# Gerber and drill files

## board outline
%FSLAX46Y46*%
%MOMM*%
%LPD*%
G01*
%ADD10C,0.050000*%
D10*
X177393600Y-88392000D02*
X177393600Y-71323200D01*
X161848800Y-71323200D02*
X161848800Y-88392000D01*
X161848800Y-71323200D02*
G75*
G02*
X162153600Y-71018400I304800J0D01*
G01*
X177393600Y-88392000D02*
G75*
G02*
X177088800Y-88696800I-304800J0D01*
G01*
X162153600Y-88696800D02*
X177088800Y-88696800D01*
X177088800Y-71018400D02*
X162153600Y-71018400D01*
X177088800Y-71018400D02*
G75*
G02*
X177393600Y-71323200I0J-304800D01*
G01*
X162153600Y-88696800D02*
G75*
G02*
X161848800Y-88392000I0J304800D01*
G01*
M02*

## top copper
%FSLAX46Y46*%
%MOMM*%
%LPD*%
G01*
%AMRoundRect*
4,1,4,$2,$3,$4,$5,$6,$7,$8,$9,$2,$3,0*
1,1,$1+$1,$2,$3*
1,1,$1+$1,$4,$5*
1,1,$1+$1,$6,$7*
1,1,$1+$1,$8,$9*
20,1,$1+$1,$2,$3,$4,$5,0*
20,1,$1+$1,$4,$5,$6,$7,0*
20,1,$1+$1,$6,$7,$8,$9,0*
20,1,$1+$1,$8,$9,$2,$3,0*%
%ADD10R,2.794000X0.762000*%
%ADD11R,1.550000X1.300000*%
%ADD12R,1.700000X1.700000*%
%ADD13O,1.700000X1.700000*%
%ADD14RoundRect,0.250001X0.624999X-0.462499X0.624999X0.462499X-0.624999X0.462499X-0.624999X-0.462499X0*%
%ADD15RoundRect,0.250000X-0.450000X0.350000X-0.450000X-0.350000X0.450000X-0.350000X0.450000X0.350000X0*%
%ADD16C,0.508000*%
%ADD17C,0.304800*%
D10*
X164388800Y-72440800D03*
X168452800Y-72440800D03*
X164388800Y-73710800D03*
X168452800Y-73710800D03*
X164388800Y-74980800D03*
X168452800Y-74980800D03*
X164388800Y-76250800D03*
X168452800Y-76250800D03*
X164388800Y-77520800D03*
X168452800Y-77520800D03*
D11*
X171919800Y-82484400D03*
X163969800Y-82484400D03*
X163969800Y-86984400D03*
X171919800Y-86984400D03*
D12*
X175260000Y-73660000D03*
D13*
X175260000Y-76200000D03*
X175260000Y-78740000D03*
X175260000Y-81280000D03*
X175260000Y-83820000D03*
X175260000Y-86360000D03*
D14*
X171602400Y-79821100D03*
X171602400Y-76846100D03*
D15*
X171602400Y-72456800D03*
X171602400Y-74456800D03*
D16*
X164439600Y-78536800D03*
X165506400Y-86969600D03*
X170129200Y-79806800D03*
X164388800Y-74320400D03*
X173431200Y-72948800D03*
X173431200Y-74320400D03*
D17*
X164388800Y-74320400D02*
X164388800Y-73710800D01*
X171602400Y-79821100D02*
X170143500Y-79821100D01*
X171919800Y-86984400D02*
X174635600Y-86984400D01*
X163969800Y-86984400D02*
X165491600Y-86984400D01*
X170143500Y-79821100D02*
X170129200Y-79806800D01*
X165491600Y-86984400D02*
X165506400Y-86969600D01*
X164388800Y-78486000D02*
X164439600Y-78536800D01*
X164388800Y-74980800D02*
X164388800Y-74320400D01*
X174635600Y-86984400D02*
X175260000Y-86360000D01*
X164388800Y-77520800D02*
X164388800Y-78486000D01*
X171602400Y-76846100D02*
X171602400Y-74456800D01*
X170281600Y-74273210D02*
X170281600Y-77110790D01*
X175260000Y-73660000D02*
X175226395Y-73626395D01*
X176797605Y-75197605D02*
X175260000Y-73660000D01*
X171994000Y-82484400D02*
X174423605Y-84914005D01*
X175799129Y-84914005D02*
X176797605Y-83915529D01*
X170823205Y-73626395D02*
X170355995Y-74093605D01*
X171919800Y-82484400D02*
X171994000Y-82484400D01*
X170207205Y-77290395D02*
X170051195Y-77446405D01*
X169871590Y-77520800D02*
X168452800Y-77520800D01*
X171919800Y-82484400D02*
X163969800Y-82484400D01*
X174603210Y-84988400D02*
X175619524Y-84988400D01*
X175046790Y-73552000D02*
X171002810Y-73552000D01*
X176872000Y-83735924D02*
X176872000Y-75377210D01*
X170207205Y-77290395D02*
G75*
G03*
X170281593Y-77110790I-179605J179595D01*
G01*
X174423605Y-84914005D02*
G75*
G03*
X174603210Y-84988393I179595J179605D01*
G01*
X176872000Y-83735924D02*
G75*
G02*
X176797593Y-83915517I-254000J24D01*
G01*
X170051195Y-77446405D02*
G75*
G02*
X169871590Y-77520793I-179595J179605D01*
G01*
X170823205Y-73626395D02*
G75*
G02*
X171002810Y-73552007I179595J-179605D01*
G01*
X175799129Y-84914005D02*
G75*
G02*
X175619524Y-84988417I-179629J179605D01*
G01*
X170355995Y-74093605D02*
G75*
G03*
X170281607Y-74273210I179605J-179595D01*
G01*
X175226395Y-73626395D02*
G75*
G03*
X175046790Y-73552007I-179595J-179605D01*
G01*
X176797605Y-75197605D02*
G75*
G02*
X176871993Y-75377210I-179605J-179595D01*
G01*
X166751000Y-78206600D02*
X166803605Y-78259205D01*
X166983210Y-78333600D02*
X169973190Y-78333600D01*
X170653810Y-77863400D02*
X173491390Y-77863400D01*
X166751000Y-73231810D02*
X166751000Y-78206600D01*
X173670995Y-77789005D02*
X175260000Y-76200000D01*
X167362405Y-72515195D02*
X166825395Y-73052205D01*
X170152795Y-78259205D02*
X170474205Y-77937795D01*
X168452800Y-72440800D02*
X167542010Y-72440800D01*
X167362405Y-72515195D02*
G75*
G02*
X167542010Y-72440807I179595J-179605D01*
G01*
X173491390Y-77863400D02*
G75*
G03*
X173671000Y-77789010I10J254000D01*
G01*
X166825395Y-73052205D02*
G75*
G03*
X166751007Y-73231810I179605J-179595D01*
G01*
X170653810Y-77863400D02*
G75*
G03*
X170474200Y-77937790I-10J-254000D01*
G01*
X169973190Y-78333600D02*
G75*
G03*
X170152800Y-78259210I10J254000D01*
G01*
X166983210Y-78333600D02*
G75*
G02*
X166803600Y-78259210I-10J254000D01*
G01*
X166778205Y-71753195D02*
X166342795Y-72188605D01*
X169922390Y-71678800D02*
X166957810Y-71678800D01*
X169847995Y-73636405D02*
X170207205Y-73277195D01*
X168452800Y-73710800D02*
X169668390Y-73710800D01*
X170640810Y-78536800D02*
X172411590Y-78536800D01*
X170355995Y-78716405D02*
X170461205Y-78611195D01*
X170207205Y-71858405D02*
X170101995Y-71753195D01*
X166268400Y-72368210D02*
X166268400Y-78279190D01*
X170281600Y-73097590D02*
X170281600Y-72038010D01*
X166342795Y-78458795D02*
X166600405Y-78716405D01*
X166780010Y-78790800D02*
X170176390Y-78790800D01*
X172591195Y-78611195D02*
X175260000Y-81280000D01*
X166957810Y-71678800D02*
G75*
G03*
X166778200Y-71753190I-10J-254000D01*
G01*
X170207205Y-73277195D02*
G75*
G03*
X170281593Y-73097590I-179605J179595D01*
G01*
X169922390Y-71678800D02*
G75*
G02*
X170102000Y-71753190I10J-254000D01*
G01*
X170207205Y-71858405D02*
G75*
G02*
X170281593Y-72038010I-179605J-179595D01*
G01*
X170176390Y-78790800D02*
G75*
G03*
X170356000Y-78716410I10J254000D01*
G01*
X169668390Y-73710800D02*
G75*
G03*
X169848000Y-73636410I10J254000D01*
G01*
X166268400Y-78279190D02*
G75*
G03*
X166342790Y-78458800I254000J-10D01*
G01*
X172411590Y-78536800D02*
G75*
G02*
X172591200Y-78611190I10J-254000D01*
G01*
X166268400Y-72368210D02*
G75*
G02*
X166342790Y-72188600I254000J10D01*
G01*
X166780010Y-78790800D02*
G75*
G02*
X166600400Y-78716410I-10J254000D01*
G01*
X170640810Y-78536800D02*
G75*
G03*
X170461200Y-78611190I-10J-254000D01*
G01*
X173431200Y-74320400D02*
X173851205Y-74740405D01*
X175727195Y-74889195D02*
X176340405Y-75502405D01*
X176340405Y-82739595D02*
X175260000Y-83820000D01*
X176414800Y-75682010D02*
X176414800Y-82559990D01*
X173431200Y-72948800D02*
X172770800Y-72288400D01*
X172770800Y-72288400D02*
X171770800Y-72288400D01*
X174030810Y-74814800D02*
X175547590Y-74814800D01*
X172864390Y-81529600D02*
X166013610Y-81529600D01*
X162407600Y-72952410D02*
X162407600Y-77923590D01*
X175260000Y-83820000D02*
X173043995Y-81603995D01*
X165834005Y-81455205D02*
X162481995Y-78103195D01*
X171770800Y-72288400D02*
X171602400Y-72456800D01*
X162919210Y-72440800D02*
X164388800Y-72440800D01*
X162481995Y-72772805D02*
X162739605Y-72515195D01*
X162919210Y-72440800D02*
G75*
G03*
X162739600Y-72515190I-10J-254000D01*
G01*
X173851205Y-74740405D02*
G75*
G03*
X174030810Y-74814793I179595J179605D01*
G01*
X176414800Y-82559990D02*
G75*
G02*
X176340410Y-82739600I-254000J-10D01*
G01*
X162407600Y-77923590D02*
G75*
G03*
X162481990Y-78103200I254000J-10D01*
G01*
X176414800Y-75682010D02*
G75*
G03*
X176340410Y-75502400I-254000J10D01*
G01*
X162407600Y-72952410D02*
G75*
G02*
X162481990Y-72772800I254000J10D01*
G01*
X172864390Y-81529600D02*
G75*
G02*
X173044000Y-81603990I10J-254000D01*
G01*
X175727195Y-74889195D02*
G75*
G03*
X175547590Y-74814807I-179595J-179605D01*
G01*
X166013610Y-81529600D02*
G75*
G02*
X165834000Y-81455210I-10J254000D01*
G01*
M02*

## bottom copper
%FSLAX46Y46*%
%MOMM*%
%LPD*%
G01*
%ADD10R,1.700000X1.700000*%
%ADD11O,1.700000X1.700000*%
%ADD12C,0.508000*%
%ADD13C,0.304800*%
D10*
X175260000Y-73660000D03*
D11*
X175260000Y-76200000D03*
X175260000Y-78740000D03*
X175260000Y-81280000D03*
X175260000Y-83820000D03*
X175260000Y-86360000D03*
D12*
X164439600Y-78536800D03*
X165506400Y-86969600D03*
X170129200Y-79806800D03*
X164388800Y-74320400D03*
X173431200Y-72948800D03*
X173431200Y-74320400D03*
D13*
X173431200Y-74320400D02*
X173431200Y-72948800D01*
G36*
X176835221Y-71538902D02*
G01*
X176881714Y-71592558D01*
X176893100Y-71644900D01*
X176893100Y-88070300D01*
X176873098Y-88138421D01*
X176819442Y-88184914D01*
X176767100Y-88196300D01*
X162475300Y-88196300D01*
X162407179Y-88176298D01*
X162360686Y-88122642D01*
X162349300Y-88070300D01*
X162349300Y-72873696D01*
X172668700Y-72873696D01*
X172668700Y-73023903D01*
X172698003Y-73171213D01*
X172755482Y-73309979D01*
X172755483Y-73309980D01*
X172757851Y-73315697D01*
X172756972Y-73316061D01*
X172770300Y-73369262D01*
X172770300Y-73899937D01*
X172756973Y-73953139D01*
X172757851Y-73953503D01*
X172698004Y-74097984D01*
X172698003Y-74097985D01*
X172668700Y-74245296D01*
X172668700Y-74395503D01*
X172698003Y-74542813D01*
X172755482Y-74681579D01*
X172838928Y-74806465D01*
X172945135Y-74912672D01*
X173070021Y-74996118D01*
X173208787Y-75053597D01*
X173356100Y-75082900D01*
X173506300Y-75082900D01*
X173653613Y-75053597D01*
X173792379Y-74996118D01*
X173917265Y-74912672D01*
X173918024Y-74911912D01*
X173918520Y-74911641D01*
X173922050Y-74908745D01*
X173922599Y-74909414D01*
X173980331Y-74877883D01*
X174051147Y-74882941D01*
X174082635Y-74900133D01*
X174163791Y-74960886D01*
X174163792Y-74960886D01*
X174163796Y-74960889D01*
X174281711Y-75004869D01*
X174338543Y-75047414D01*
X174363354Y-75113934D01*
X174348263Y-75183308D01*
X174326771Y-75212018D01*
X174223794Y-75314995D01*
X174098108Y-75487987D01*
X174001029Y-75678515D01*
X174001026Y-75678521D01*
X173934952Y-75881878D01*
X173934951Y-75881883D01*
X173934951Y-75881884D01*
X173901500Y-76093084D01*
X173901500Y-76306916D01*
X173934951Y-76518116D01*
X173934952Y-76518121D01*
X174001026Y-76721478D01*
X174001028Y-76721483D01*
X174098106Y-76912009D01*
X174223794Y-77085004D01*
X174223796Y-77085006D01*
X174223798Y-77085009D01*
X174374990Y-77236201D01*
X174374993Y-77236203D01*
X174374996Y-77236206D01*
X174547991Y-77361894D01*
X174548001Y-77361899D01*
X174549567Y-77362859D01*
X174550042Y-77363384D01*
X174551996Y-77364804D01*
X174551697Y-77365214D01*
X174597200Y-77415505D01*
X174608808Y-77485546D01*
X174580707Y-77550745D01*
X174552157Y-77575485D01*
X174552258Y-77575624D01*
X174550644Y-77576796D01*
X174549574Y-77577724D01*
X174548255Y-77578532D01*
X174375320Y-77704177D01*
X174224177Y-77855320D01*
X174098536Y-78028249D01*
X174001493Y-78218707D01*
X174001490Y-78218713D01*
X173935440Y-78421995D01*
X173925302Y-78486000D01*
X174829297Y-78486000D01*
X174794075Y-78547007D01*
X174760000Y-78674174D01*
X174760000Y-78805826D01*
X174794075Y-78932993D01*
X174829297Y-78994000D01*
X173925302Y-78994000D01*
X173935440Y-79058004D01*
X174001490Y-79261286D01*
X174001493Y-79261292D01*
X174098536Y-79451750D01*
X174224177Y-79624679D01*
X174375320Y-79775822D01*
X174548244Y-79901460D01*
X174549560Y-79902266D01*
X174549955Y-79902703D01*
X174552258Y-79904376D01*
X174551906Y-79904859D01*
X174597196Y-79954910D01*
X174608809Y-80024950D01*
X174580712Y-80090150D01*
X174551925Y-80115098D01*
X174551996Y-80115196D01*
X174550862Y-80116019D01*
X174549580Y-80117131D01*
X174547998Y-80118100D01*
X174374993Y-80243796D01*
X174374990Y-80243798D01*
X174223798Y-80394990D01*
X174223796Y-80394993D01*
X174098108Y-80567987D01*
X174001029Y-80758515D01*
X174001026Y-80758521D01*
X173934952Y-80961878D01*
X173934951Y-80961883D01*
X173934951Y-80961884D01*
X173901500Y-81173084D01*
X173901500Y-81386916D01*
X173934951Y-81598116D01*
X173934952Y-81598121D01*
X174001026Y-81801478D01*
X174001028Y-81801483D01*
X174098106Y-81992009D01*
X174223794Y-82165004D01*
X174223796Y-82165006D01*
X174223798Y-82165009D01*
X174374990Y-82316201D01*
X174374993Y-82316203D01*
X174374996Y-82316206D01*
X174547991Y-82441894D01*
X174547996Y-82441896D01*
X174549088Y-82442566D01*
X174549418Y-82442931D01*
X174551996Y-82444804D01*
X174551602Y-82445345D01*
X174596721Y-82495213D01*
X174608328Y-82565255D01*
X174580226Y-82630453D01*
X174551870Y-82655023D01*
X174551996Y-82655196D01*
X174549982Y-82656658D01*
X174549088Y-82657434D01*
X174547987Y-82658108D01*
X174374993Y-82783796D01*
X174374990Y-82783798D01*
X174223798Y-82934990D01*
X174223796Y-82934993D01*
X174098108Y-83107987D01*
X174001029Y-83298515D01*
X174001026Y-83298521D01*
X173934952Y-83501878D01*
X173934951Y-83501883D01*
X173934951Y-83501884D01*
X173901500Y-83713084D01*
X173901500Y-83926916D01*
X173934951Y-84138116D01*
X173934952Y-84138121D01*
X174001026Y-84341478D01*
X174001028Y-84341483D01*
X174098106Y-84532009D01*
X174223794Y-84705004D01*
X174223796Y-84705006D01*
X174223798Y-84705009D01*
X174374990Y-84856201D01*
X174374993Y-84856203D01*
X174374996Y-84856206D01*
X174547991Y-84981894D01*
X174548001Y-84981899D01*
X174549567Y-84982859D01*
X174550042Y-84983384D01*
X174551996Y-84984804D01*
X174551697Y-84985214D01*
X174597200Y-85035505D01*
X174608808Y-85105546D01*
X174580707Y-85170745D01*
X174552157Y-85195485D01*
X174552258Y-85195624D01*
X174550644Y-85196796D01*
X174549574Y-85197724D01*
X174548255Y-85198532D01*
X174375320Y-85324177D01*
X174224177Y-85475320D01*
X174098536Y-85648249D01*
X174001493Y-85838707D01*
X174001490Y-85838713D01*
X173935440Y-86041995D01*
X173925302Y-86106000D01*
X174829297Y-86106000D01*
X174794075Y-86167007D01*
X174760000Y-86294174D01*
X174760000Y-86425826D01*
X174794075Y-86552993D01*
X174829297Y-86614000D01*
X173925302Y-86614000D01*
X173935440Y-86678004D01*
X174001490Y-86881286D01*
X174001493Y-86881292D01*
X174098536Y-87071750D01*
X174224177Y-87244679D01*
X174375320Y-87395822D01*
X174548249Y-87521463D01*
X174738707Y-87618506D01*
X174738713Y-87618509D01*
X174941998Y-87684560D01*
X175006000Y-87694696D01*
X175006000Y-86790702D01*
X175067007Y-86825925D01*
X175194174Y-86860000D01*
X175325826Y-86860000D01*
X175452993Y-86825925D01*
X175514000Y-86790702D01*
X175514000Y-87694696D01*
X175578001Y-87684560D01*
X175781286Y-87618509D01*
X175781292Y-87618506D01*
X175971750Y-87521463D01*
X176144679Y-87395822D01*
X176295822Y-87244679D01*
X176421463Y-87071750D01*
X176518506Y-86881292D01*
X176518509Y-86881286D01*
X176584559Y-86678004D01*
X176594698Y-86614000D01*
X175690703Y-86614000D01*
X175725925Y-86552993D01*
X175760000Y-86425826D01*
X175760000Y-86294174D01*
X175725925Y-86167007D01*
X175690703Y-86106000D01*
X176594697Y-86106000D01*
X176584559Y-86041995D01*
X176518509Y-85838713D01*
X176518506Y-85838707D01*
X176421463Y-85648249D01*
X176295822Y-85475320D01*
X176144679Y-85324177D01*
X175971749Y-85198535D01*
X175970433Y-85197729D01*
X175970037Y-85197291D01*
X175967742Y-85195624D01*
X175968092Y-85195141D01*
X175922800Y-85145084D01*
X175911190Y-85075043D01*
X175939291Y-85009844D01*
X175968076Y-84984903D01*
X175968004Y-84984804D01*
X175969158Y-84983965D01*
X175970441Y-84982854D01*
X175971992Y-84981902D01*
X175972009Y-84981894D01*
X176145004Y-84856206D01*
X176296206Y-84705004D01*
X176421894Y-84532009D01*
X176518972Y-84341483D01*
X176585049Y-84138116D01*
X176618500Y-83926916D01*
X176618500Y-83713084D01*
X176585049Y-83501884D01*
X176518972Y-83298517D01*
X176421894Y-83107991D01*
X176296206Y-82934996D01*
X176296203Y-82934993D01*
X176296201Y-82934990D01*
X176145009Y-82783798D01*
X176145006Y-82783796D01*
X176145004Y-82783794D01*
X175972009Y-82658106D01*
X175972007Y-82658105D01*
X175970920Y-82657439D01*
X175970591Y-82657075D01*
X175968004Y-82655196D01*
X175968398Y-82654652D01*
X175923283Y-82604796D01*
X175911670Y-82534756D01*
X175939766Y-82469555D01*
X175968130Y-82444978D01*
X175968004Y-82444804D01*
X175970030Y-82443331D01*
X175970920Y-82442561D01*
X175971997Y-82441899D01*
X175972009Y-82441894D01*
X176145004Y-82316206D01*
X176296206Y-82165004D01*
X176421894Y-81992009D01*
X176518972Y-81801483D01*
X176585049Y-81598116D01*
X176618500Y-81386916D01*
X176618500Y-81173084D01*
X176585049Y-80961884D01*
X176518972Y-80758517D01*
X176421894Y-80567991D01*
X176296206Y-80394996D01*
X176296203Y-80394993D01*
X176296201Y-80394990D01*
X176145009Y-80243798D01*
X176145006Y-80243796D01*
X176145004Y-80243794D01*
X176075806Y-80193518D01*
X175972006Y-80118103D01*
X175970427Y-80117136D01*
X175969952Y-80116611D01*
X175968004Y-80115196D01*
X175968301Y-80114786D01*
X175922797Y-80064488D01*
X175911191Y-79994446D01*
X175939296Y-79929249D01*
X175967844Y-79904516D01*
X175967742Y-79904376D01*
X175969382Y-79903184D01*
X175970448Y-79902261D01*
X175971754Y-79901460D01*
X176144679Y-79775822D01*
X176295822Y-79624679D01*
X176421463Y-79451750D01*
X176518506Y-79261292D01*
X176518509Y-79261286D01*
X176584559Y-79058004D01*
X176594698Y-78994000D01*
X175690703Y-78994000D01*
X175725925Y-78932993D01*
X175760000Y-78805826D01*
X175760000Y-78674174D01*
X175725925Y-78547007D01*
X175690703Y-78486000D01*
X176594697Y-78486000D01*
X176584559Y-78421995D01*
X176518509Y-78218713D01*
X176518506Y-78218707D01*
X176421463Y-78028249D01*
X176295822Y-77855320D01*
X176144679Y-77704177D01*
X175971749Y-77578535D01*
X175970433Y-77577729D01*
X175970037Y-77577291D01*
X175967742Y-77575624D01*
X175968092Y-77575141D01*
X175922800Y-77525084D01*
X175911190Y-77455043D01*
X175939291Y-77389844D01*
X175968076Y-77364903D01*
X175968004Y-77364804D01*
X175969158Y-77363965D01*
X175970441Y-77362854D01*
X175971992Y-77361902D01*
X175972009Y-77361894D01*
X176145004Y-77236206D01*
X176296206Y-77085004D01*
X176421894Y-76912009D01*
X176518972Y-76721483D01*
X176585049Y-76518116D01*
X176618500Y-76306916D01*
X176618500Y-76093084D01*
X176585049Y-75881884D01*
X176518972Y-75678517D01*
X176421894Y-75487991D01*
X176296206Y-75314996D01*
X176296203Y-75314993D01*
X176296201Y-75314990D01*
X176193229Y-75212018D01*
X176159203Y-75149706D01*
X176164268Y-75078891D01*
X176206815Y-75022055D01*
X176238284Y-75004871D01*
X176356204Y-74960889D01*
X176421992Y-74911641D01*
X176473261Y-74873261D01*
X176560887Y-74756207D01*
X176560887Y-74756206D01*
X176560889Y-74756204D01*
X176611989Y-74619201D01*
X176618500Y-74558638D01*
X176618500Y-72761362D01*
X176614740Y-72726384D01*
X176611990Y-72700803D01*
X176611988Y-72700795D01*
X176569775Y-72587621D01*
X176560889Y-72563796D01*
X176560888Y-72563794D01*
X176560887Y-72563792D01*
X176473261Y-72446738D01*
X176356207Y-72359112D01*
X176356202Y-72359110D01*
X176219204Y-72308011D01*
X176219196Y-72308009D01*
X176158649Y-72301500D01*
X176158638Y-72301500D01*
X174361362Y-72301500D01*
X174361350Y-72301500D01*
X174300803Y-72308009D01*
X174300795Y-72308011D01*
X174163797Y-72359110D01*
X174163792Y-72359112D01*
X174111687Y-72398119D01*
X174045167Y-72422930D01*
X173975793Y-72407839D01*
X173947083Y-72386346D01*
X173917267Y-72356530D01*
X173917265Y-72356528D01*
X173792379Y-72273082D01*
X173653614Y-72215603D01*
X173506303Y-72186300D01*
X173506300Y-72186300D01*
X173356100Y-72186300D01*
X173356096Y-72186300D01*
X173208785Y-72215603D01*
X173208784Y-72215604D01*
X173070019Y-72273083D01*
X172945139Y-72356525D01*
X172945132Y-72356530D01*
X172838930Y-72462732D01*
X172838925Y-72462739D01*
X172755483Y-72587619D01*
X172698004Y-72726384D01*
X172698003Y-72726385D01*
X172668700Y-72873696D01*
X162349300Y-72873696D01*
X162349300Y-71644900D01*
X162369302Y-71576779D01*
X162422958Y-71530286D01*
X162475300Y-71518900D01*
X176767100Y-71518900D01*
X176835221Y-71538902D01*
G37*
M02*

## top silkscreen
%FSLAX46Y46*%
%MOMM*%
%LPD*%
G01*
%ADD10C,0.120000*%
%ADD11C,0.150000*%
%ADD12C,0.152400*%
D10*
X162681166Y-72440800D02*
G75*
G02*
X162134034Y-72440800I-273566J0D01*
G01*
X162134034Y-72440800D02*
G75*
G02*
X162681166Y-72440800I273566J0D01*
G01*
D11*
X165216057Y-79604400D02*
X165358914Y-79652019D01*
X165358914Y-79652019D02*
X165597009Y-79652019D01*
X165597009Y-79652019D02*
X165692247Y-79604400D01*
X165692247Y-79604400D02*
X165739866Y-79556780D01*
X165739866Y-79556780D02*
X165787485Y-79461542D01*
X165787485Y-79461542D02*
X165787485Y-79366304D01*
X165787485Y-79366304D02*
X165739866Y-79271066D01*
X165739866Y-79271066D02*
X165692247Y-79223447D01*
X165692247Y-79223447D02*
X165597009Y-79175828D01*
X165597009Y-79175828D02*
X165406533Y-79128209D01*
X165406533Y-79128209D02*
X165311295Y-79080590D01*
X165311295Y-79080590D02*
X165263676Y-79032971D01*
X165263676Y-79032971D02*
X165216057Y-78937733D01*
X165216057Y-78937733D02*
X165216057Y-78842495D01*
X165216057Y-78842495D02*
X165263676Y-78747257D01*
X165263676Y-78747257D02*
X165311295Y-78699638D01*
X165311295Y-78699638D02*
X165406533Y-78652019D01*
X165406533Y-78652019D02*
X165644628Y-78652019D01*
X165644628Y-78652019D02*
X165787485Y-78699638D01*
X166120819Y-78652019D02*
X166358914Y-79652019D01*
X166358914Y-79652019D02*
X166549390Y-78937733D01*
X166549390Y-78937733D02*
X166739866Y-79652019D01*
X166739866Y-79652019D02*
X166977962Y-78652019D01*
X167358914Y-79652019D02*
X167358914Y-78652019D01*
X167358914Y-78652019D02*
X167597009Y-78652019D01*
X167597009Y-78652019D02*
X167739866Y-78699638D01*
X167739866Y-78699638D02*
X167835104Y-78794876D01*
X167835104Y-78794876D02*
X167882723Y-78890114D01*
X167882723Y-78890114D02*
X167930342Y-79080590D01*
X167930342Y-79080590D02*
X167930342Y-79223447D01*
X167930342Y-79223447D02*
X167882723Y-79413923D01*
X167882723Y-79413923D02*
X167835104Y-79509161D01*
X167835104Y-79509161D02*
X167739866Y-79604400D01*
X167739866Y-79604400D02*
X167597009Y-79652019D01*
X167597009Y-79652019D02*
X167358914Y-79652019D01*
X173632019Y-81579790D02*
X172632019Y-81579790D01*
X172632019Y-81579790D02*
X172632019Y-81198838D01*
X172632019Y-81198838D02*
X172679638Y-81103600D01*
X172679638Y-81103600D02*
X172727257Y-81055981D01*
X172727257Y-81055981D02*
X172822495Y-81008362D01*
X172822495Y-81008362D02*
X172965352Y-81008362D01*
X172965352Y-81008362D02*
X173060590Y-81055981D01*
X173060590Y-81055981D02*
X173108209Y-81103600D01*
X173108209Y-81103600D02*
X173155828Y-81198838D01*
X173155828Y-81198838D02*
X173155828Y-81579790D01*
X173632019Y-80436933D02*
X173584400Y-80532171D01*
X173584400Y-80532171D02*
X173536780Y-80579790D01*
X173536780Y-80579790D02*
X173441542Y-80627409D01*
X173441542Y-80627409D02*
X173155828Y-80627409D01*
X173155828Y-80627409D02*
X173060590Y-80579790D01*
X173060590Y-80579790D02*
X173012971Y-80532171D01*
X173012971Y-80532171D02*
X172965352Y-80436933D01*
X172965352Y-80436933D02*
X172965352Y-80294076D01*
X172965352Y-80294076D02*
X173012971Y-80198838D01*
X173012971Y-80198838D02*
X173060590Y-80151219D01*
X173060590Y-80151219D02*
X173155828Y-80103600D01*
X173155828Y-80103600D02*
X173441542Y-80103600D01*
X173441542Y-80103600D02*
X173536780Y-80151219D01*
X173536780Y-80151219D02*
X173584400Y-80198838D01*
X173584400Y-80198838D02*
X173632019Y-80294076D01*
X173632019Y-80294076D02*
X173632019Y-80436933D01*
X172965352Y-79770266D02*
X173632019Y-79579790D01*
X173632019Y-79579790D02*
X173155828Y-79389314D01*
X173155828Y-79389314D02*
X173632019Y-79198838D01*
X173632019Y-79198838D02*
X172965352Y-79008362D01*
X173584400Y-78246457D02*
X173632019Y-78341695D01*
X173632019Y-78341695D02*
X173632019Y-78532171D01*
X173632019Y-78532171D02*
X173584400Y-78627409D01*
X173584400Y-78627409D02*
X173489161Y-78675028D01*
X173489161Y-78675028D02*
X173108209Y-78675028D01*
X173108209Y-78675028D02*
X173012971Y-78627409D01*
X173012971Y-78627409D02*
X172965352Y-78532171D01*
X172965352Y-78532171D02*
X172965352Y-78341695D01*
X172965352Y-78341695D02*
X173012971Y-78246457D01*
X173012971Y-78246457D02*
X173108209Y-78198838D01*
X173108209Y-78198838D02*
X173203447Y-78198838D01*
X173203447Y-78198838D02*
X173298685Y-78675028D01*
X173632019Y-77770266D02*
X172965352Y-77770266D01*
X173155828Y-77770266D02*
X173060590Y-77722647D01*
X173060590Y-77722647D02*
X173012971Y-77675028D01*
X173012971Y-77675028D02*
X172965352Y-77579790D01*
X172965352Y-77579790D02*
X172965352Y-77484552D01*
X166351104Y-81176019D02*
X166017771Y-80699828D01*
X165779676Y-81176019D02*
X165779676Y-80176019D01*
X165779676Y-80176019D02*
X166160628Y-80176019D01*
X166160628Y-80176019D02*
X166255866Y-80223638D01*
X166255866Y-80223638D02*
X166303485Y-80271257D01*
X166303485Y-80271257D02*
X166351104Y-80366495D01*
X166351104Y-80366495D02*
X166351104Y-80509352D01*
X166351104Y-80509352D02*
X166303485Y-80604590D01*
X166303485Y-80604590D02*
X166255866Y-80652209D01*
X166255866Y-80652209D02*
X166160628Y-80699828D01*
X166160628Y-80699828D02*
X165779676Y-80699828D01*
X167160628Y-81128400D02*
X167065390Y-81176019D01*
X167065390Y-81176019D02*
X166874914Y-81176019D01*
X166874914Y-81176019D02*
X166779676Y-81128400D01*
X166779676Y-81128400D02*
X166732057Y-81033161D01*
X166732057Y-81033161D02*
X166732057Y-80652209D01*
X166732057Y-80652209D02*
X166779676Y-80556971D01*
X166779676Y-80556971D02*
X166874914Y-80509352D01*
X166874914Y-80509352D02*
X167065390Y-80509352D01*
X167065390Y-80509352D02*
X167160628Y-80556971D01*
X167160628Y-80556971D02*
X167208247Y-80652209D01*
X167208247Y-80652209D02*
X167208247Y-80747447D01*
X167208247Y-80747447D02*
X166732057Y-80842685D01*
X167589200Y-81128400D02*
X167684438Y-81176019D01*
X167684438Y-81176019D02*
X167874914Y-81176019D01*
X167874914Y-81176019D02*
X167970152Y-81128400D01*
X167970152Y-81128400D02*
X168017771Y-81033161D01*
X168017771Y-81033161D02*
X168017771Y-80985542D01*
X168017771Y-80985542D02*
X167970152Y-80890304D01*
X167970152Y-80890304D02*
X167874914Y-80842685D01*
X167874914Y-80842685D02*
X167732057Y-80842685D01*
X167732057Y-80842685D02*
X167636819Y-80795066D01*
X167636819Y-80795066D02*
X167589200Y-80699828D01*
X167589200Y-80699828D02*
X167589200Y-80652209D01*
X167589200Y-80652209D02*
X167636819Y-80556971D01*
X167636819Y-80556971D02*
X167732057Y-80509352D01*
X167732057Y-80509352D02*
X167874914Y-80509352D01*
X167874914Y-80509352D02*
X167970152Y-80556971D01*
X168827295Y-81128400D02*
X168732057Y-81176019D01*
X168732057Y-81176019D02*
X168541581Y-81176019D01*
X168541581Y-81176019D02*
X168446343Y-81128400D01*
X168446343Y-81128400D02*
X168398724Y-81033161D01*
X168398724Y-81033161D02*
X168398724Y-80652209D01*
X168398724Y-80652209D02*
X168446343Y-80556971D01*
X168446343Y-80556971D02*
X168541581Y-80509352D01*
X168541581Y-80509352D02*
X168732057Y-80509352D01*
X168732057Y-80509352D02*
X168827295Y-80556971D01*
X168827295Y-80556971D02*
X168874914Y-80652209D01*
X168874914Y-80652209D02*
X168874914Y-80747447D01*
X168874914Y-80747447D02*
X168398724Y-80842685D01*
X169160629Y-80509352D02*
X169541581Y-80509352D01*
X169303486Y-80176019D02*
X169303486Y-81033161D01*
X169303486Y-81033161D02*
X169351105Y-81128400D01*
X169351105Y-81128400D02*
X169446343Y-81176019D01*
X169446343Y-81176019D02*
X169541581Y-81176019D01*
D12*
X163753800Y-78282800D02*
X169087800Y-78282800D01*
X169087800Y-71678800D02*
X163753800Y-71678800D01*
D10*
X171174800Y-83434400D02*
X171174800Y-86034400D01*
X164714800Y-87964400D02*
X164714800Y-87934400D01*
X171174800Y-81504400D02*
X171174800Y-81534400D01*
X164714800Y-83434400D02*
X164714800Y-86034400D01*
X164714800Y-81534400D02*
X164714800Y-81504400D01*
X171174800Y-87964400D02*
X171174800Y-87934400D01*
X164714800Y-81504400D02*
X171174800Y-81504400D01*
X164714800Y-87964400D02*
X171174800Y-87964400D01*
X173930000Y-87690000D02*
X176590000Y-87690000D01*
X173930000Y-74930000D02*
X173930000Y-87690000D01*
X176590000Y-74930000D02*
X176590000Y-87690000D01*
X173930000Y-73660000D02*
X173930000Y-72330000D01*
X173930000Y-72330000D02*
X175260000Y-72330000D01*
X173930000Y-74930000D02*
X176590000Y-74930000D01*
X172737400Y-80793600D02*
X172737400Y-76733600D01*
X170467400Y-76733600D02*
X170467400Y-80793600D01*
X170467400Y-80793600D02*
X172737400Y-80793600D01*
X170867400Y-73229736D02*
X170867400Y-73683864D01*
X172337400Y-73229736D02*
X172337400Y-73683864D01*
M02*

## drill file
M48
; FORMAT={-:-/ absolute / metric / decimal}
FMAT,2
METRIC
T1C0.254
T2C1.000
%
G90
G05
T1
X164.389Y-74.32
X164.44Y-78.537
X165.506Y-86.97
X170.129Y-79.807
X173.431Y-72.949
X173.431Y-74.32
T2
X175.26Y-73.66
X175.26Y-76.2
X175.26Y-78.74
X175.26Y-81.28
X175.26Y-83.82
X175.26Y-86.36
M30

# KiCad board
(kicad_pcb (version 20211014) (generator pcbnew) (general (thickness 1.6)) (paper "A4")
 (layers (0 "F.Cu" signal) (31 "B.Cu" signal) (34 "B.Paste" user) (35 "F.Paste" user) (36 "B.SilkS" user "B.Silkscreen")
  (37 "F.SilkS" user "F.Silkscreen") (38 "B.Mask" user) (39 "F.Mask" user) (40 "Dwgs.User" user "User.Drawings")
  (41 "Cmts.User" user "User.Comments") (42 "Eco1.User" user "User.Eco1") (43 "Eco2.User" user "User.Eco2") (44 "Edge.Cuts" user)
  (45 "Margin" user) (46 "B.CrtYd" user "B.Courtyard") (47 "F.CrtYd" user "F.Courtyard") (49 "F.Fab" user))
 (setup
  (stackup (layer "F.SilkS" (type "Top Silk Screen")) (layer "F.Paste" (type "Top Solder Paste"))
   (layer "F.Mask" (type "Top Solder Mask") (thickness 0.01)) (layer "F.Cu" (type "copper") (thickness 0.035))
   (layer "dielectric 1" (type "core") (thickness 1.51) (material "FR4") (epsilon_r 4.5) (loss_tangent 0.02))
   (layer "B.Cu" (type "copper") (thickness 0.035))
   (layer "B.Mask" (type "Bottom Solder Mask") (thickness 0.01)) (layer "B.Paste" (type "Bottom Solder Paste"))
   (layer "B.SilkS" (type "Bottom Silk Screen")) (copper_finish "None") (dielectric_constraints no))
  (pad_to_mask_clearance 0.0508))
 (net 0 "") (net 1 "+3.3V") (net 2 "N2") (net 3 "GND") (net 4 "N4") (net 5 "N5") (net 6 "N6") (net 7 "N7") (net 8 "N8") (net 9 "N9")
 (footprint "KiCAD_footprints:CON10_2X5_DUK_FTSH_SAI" (layer "F.Cu") (at 166.4208 74.9808 -90)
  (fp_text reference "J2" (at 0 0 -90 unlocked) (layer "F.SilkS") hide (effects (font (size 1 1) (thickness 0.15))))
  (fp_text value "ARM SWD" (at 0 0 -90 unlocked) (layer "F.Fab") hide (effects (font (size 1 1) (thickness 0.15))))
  (fp_line (start 3.302 2.667) (end 3.302 -2.667) (layer "F.SilkS") (width 0.1524))
  (fp_line (start -3.302 -2.667) (end -3.302 2.667) (layer "F.SilkS") (width 0.1524))
  (pad "1" smd rect (at -2.54 2.032 270) (size 0.762 2.794) (layers "F.Cu" "F.Paste" "F.Mask") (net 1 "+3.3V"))
  (pad "2" smd rect (at -2.54 -2.032 270) (size 0.762 2.794) (layers "F.Cu" "F.Paste" "F.Mask") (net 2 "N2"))
  (pad "3" smd rect (at -1.27 2.032 270) (size 0.762 2.794) (layers "F.Cu" "F.Paste" "F.Mask") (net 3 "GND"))
  (pad "4" smd rect (at -1.27 -2.032 270) (size 0.762 2.794) (layers "F.Cu" "F.Paste" "F.Mask") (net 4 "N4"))
  (pad "5" smd rect (at 0 2.032 270) (size 0.762 2.794) (layers "F.Cu" "F.Paste" "F.Mask") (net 3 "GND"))
  (pad "6" smd rect (at 0 -2.032 270) (size 0.762 2.794) (layers "F.Cu" "F.Paste" "F.Mask") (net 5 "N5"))
  (pad "7" smd rect (at 1.27 2.032 270) (size 0.762 2.794) (layers "F.Cu" "F.Paste" "F.Mask") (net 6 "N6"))
  (pad "8" smd rect (at 1.27 -2.032 270) (size 0.762 2.794) (layers "F.Cu" "F.Paste" "F.Mask") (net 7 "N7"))
  (pad "9" smd rect (at 2.54 2.032 270) (size 0.762 2.794) (layers "F.Cu" "F.Paste" "F.Mask") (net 3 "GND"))
  (pad "10" smd rect (at 2.54 -2.032 270) (size 0.762 2.794) (layers "F.Cu" "F.Paste" "F.Mask") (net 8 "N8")))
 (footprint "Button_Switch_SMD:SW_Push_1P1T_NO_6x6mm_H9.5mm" (layer "F.Cu") (at 167.9448 84.7344)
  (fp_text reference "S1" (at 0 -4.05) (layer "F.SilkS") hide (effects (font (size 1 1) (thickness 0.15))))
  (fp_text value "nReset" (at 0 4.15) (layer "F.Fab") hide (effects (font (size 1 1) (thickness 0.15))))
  (fp_line (start 3.23 -1.3) (end 3.23 1.3) (layer "F.SilkS") (width 0.12))
  (fp_line (start -3.23 3.23) (end -3.23 3.2) (layer "F.SilkS") (width 0.12))
  (fp_line (start 3.23 -3.23) (end 3.23 -3.2) (layer "F.SilkS") (width 0.12))
  (fp_line (start -3.23 -1.3) (end -3.23 1.3) (layer "F.SilkS") (width 0.12))
  (fp_line (start -3.23 -3.2) (end -3.23 -3.23) (layer "F.SilkS") (width 0.12))
  (fp_line (start 3.23 3.23) (end 3.23 3.2) (layer "F.SilkS") (width 0.12))
  (fp_line (start -3.23 -3.23) (end 3.23 -3.23) (layer "F.SilkS") (width 0.12))
  (fp_line (start -3.23 3.23) (end 3.23 3.23) (layer "F.SilkS") (width 0.12))
  (pad "1" smd rect (at 3.975 -2.25) (size 1.55 1.3) (layers "F.Cu" "F.Paste" "F.Mask") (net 8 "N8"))
  (pad "1" smd rect (at -3.975 -2.25) (size 1.55 1.3) (layers "F.Cu" "F.Paste" "F.Mask") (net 8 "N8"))
  (pad "2" smd rect (at -3.975 2.25) (size 1.55 1.3) (layers "F.Cu" "F.Paste" "F.Mask") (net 3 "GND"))
  (pad "2" smd rect (at 3.975 2.25) (size 1.55 1.3) (layers "F.Cu" "F.Paste" "F.Mask") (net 3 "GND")))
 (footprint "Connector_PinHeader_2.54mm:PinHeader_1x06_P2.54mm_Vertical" (layer "F.Cu") (at 175.26 73.66)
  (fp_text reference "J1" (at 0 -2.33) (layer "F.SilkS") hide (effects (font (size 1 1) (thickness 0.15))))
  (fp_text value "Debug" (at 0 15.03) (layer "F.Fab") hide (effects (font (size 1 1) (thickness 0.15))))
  (fp_line (start -1.33 14.03) (end 1.33 14.03) (layer "F.SilkS") (width 0.12))
  (fp_line (start -1.33 1.27) (end -1.33 14.03) (layer "F.SilkS") (width 0.12))
  (fp_line (start 1.33 1.27) (end 1.33 14.03) (layer "F.SilkS") (width 0.12))
  (fp_line (start -1.33 0) (end -1.33 -1.33) (layer "F.SilkS") (width 0.12))
  (fp_line (start -1.33 -1.33) (end 0 -1.33) (layer "F.SilkS") (width 0.12))
  (fp_line (start -1.33 1.27) (end 1.33 1.27) (layer "F.SilkS") (width 0.12))
  (pad "1" thru_hole rect (at 0 0) (size 1.7 1.7) (drill 1) (layers *.Cu *.Mask) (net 8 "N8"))
  (pad "2" thru_hole oval (at 0 2.54) (size 1.7 1.7) (drill 1) (layers *.Cu *.Mask) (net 2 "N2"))
  (pad "3" thru_hole oval (at 0 5.08) (size 1.7 1.7) (drill 1) (layers *.Cu *.Mask) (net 3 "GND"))
  (pad "4" thru_hole oval (at 0 7.62) (size 1.7 1.7) (drill 1) (layers *.Cu *.Mask) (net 4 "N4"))
  (pad "5" thru_hole oval (at 0 10.16) (size 1.7 1.7) (drill 1) (layers *.Cu *.Mask) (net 1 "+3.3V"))
  (pad "6" thru_hole oval (at 0 12.7) (size 1.7 1.7) (drill 1) (layers *.Cu *.Mask) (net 3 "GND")))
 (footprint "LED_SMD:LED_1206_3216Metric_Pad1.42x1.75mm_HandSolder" (layer "F.Cu") (at 171.6024 78.3336 90)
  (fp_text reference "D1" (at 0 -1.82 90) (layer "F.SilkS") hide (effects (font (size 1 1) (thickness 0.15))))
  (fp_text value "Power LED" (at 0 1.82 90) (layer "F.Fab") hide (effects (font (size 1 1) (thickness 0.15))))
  (fp_line (start -2.46 1.135) (end 1.6 1.135) (layer "F.SilkS") (width 0.12))
  (fp_line (start 1.6 -1.135) (end -2.46 -1.135) (layer "F.SilkS") (width 0.12))
  (fp_line (start -2.46 -1.135) (end -2.46 1.135) (layer "F.SilkS") (width 0.12))
  (pad "1" smd roundrect (at -1.4875 0 90) (size 1.425 1.75) (layers "F.Cu" "F.Paste" "F.Mask") (roundrect_rratio 0.175439) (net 3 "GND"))
  (pad "2" smd roundrect (at 1.4875 0 90) (size 1.425 1.75) (layers "F.Cu" "F.Paste" "F.Mask") (roundrect_rratio 0.175439) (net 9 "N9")))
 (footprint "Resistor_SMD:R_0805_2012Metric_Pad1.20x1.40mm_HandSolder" (layer "F.Cu") (at 171.6024 73.4568 -90)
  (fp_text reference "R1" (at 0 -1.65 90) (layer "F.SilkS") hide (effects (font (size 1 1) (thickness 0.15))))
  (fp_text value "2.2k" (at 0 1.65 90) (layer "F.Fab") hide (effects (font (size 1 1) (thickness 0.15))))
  (fp_line (start -0.227064 0.735) (end 0.227064 0.735) (layer "F.SilkS") (width 0.12))
  (fp_line (start -0.227064 -0.735) (end 0.227064 -0.735) (layer "F.SilkS") (width 0.12))
  (pad "1" smd roundrect (at -1 0 270) (size 1.2 1.4) (layers "F.Cu" "F.Paste" "F.Mask") (roundrect_rratio 0.208333) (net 1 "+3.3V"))
  (pad "2" smd roundrect (at 1 0 270) (size 1.2 1.4) (layers "F.Cu" "F.Paste" "F.Mask") (roundrect_rratio 0.208333) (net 9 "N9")))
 (gr_circle (center 162.4076 72.4408) (end 162.5092 72.1868) (layer "F.SilkS") (width 0.12) (fill none))
 (gr_line (start 177.3936 88.392) (end 177.3936 71.3232) (layer "Edge.Cuts") (width 0.05))
 (gr_line (start 161.8488 71.3232) (end 161.8488 88.392) (layer "Edge.Cuts") (width 0.05))
 (gr_arc (start 161.8488 71.3232) (mid 161.938074 71.107674) (end 162.1536 71.0184) (layer "Edge.Cuts") (width 0.05))
 (gr_arc (start 177.3936 88.392) (mid 177.304326 88.607526) (end 177.0888 88.6968) (layer "Edge.Cuts") (width 0.05))
 (gr_line (start 162.1536 88.6968) (end 177.0888 88.6968) (layer "Edge.Cuts") (width 0.05))
 (gr_line (start 177.0888 71.0184) (end 162.1536 71.0184) (layer "Edge.Cuts") (width 0.05))
 (gr_arc (start 177.0888 71.0184) (mid 177.304326 71.107674) (end 177.3936 71.3232) (layer "Edge.Cuts") (width 0.05))
 (gr_arc (start 162.1536 88.6968) (mid 161.938074 88.607526) (end 161.8488 88.392) (layer "Edge.Cuts") (width 0.05))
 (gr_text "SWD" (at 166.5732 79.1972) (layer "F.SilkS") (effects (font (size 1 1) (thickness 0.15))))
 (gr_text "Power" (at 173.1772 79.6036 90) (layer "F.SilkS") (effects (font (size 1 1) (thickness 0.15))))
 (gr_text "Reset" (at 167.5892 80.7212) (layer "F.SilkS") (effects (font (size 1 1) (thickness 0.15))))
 (segment (start 164.3888 74.3204) (end 164.3888 73.7108) (width 0.3048) (layer "F.Cu") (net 3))
 (segment (start 171.6024 79.8211) (end 170.1435 79.8211) (width 0.3048) (layer "F.Cu") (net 3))
 (segment (start 171.9198 86.9844) (end 174.6356 86.9844) (width 0.3048) (layer "F.Cu") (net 3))
 (segment (start 163.9698 86.9844) (end 165.4916 86.9844) (width 0.3048) (layer "F.Cu") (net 3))
 (segment (start 170.1435 79.8211) (end 170.1292 79.8068) (width 0.3048) (layer "F.Cu") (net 3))
 (segment (start 165.4916 86.9844) (end 165.5064 86.9696) (width 0.3048) (layer "F.Cu") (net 3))
 (segment (start 164.3888 78.486) (end 164.4396 78.5368) (width 0.3048) (layer "F.Cu") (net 3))
 (segment (start 164.3888 74.9808) (end 164.3888 74.3204) (width 0.3048) (layer "F.Cu") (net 3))
 (segment (start 174.6356 86.9844) (end 175.26 86.36) (width 0.3048) (layer "F.Cu") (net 3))
 (segment (start 164.3888 77.5208) (end 164.3888 78.486) (width 0.3048) (layer "F.Cu") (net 3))
 (via (at 164.4396 78.5368) (size 0.508) (drill 0.254) (layers "F.Cu" "B.Cu") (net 3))
 (via (at 165.5064 86.9696) (size 0.508) (drill 0.254) (layers "F.Cu" "B.Cu") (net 3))
 (via (at 170.1292 79.8068) (size 0.508) (drill 0.254) (layers "F.Cu" "B.Cu") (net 3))
 (via (at 164.3888 74.3204) (size 0.508) (drill 0.254) (layers "F.Cu" "B.Cu") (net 3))
 (segment (start 171.6024 76.8461) (end 171.6024 74.4568) (width 0.3048) (layer "F.Cu") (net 9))
 (segment (start 170.2816 74.27321) (end 170.2816 77.11079) (width 0.3048) (layer "F.Cu") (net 8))
 (segment (start 175.26 73.66) (end 175.226395 73.626395) (width 0.3048) (layer "F.Cu") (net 8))
 (segment (start 176.797605 75.197605) (end 175.26 73.66) (width 0.3048) (layer "F.Cu") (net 8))
 (segment (start 171.994 82.4844) (end 174.423605 84.914005) (width 0.3048) (layer "F.Cu") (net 8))
 (segment (start 175.799129 84.914005) (end 176.797605 83.915529) (width 0.3048) (layer "F.Cu") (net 8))
 (segment (start 170.823205 73.626395) (end 170.355995 74.093605) (width 0.3048) (layer "F.Cu") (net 8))
 (segment (start 171.9198 82.4844) (end 171.994 82.4844) (width 0.3048) (layer "F.Cu") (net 8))
 (segment (start 170.207205 77.290395) (end 170.051195 77.446405) (width 0.3048) (layer "F.Cu") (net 8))
 (segment (start 169.87159 77.5208) (end 168.4528 77.5208) (width 0.3048) (layer "F.Cu") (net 8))
 (segment (start 171.9198 82.4844) (end 163.9698 82.4844) (width 0.3048) (layer "F.Cu") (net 8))
 (segment (start 174.60321 84.9884) (end 175.619524 84.9884) (width 0.3048) (layer "F.Cu") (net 8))
 (segment (start 175.04679 73.552) (end 171.00281 73.552) (width 0.3048) (layer "F.Cu") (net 8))
 (segment (start 176.872 83.735924) (end 176.872 75.37721) (width 0.3048) (layer "F.Cu") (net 8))
 (arc (start 170.207205 77.290395) (mid 170.262265 77.207992) (end 170.2816 77.11079) (width 0.3048) (layer "F.Cu") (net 8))
 (arc (start 174.423605 84.914005) (mid 174.506008 84.969065) (end 174.60321 84.9884) (width 0.3048) (layer "F.Cu") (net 8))
 (arc (start 176.872 83.735924) (mid 176.852665 83.833126) (end 176.797605 83.915529) (width 0.3048) (layer "F.Cu") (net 8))
 (arc (start 170.051195 77.446405) (mid 169.968792 77.501465) (end 169.87159 77.5208) (width 0.3048) (layer "F.Cu") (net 8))
 (arc (start 170.823205 73.626395) (mid 170.905608 73.571335) (end 171.00281 73.552) (width 0.3048) (layer "F.Cu") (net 8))
 (arc (start 175.799129 84.914005) (mid 175.716726 84.969065) (end 175.619524 84.9884) (width 0.3048) (layer "F.Cu") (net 8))
 (arc (start 170.355995 74.093605) (mid 170.300935 74.176008) (end 170.2816 74.27321) (width 0.3048) (layer "F.Cu") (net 8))
 (arc (start 175.226395 73.626395) (mid 175.143992 73.571335) (end 175.04679 73.552) (width 0.3048) (layer "F.Cu") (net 8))
 (arc (start 176.797605 75.197605) (mid 176.852665 75.280008) (end 176.872 75.37721) (width 0.3048) (layer "F.Cu") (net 8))
 (segment (start 166.751 78.2066) (end 166.803605 78.259205) (width 0.3048) (layer "F.Cu") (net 2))
 (segment (start 166.98321 78.3336) (end 169.97319 78.3336) (width 0.3048) (layer "F.Cu") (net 2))
 (segment (start 170.65381 77.8634) (end 173.49139 77.8634) (width 0.3048) (layer "F.Cu") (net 2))
 (segment (start 166.751 73.23181) (end 166.751 78.2066) (width 0.3048) (layer "F.Cu") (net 2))
 (segment (start 173.670995 77.789005) (end 175.26 76.2) (width 0.3048) (layer "F.Cu") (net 2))
 (segment (start 167.362405 72.515195) (end 166.825395 73.052205) (width 0.3048) (layer "F.Cu") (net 2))
 (segment (start 170.152795 78.259205) (end 170.474205 77.937795) (width 0.3048) (layer "F.Cu") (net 2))
 (segment (start 168.4528 72.4408) (end 167.54201 72.4408) (width 0.3048) (layer "F.Cu") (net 2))
 (arc (start 167.362405 72.515195) (mid 167.444808 72.460135) (end 167.54201 72.4408) (width 0.3048) (layer "F.Cu") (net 2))
 (arc (start 173.49139 77.8634) (mid 173.588592 77.844065) (end 173.670995 77.789005) (width 0.3048) (layer "F.Cu") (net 2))
 (arc (start 166.825395 73.052205) (mid 166.770335 73.134608) (end 166.751 73.23181) (width 0.3048) (layer "F.Cu") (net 2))
 (arc (start 170.65381 77.8634) (mid 170.556608 77.882735) (end 170.474205 77.937795) (width 0.3048) (layer "F.Cu") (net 2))
 (arc (start 169.97319 78.3336) (mid 170.070392 78.314265) (end 170.152795 78.259205) (width 0.3048) (layer "F.Cu") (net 2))
 (arc (start 166.98321 78.3336) (mid 166.886008 78.314265) (end 166.803605 78.259205) (width 0.3048) (layer "F.Cu") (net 2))
 (segment (start 166.778205 71.753195) (end 166.342795 72.188605) (width 0.3048) (layer "F.Cu") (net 4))
 (segment (start 169.92239 71.6788) (end 166.95781 71.6788) (width 0.3048) (layer "F.Cu") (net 4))
 (segment (start 169.847995 73.636405) (end 170.207205 73.277195) (width 0.3048) (layer "F.Cu") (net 4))
 (segment (start 168.4528 73.7108) (end 169.66839 73.7108) (width 0.3048) (layer "F.Cu") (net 4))
 (segment (start 170.64081 78.5368) (end 172.41159 78.5368) (width 0.3048) (layer "F.Cu") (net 4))
 (segment (start 170.355995 78.716405) (end 170.461205 78.611195) (width 0.3048) (layer "F.Cu") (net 4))
 (segment (start 170.207205 71.858405) (end 170.101995 71.753195) (width 0.3048) (layer "F.Cu") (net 4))
 (segment (start 166.2684 72.36821) (end 166.2684 78.27919) (width 0.3048) (layer "F.Cu") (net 4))
 (segment (start 170.2816 73.09759) (end 170.2816 72.03801) (width 0.3048) (layer "F.Cu") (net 4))
 (segment (start 166.342795 78.458795) (end 166.600405 78.716405) (width 0.3048) (layer "F.Cu") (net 4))
 (segment (start 166.78001 78.7908) (end 170.17639 78.7908) (width 0.3048) (layer "F.Cu") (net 4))
 (segment (start 172.591195 78.611195) (end 175.26 81.28) (width 0.3048) (layer "F.Cu") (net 4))
 (arc (start 166.95781 71.6788) (mid 166.860608 71.698135) (end 166.778205 71.753195) (width 0.3048) (layer "F.Cu") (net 4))
 (arc (start 170.207205 73.277195) (mid 170.262265 73.194792) (end 170.2816 73.09759) (width 0.3048) (layer "F.Cu") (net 4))
 (arc (start 169.92239 71.6788) (mid 170.019592 71.698135) (end 170.101995 71.753195) (width 0.3048) (layer "F.Cu") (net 4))
 (arc (start 170.207205 71.858405) (mid 170.262265 71.940808) (end 170.2816 72.03801) (width 0.3048) (layer "F.Cu") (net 4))
 (arc (start 170.17639 78.7908) (mid 170.273592 78.771465) (end 170.355995 78.716405) (width 0.3048) (layer "F.Cu") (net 4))
 (arc (start 169.66839 73.7108) (mid 169.765592 73.691465) (end 169.847995 73.636405) (width 0.3048) (layer "F.Cu") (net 4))
 (arc (start 166.2684 78.27919) (mid 166.287735 78.376392) (end 166.342795 78.458795) (width 0.3048) (layer "F.Cu") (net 4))
 (arc (start 172.41159 78.5368) (mid 172.508792 78.556135) (end 172.591195 78.611195) (width 0.3048) (layer "F.Cu") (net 4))
 (arc (start 166.2684 72.36821) (mid 166.287735 72.271008) (end 166.342795 72.188605) (width 0.3048) (layer "F.Cu") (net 4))
 (arc (start 166.78001 78.7908) (mid 166.682808 78.771465) (end 166.600405 78.716405) (width 0.3048) (layer "F.Cu") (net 4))
 (arc (start 170.64081 78.5368) (mid 170.543608 78.556135) (end 170.461205 78.611195) (width 0.3048) (layer "F.Cu") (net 4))
 (segment (start 173.4312 74.3204) (end 173.851205 74.740405) (width 0.3048) (layer "F.Cu") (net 1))
 (segment (start 175.727195 74.889195) (end 176.340405 75.502405) (width 0.3048) (layer "F.Cu") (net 1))
 (segment (start 176.340405 82.739595) (end 175.26 83.82) (width 0.3048) (layer "F.Cu") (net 1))
 (segment (start 176.4148 75.68201) (end 176.4148 82.55999) (width 0.3048) (layer "F.Cu") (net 1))
 (segment (start 173.4312 72.9488) (end 172.7708 72.2884) (width 0.3048) (layer "F.Cu") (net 1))
 (segment (start 172.7708 72.2884) (end 171.7708 72.2884) (width 0.3048) (layer "F.Cu") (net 1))
 (segment (start 174.03081 74.8148) (end 175.54759 74.8148) (width 0.3048) (layer "F.Cu") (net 1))
 (segment (start 172.86439 81.5296) (end 166.01361 81.5296) (width 0.3048) (layer "F.Cu") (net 1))
 (segment (start 162.4076 72.95241) (end 162.4076 77.92359) (width 0.3048) (layer "F.Cu") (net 1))
 (segment (start 175.26 83.82) (end 173.043995 81.603995) (width 0.3048) (layer "F.Cu") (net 1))
 (segment (start 165.834005 81.455205) (end 162.481995 78.103195) (width 0.3048) (layer "F.Cu") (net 1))
 (segment (start 171.7708 72.2884) (end 171.6024 72.4568) (width 0.3048) (layer "F.Cu") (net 1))
 (segment (start 162.91921 72.4408) (end 164.3888 72.4408) (width 0.3048) (layer "F.Cu") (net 1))
 (segment (start 162.481995 72.772805) (end 162.739605 72.515195) (width 0.3048) (layer "F.Cu") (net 1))
 (via (at 173.4312 72.9488) (size 0.508) (drill 0.254) (layers "F.Cu" "B.Cu") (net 1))
 (via (at 173.4312 74.3204) (size 0.508) (drill 0.254) (layers "F.Cu" "B.Cu") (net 1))
 (arc (start 162.91921 72.4408) (mid 162.822008 72.460135) (end 162.739605 72.515195) (width 0.3048) (layer "F.Cu") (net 1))
 (arc (start 173.851205 74.740405) (mid 173.933608 74.795465) (end 174.03081 74.8148) (width 0.3048) (layer "F.Cu") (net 1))
 (arc (start 176.4148 82.55999) (mid 176.395465 82.657192) (end 176.340405 82.739595) (width 0.3048) (layer "F.Cu") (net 1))
 (arc (start 162.4076 77.92359) (mid 162.426935 78.020792) (end 162.481995 78.103195) (width 0.3048) (layer "F.Cu") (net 1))
 (arc (start 176.4148 75.68201) (mid 176.395465 75.584808) (end 176.340405 75.502405) (width 0.3048) (layer "F.Cu") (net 1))
 (arc (start 162.4076 72.95241) (mid 162.426935 72.855208) (end 162.481995 72.772805) (width 0.3048) (layer "F.Cu") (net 1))
 (arc (start 172.86439 81.5296) (mid 172.961592 81.548935) (end 173.043995 81.603995) (width 0.3048) (layer "F.Cu") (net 1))
 (arc (start 175.727195 74.889195) (mid 175.644792 74.834135) (end 175.54759 74.8148) (width 0.3048) (layer "F.Cu") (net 1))
 (arc (start 166.01361 81.5296) (mid 165.916408 81.510265) (end 165.834005 81.455205) (width 0.3048) (layer "F.Cu") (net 1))
 (segment (start 173.4312 74.3204) (end 173.4312 72.9488) (width 0.3048) (layer "B.Cu") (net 1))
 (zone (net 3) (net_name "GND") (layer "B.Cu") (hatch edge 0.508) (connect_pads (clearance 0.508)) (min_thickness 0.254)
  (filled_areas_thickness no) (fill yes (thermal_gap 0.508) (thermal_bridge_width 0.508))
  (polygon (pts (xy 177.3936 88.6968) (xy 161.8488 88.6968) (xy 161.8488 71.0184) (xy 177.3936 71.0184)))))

